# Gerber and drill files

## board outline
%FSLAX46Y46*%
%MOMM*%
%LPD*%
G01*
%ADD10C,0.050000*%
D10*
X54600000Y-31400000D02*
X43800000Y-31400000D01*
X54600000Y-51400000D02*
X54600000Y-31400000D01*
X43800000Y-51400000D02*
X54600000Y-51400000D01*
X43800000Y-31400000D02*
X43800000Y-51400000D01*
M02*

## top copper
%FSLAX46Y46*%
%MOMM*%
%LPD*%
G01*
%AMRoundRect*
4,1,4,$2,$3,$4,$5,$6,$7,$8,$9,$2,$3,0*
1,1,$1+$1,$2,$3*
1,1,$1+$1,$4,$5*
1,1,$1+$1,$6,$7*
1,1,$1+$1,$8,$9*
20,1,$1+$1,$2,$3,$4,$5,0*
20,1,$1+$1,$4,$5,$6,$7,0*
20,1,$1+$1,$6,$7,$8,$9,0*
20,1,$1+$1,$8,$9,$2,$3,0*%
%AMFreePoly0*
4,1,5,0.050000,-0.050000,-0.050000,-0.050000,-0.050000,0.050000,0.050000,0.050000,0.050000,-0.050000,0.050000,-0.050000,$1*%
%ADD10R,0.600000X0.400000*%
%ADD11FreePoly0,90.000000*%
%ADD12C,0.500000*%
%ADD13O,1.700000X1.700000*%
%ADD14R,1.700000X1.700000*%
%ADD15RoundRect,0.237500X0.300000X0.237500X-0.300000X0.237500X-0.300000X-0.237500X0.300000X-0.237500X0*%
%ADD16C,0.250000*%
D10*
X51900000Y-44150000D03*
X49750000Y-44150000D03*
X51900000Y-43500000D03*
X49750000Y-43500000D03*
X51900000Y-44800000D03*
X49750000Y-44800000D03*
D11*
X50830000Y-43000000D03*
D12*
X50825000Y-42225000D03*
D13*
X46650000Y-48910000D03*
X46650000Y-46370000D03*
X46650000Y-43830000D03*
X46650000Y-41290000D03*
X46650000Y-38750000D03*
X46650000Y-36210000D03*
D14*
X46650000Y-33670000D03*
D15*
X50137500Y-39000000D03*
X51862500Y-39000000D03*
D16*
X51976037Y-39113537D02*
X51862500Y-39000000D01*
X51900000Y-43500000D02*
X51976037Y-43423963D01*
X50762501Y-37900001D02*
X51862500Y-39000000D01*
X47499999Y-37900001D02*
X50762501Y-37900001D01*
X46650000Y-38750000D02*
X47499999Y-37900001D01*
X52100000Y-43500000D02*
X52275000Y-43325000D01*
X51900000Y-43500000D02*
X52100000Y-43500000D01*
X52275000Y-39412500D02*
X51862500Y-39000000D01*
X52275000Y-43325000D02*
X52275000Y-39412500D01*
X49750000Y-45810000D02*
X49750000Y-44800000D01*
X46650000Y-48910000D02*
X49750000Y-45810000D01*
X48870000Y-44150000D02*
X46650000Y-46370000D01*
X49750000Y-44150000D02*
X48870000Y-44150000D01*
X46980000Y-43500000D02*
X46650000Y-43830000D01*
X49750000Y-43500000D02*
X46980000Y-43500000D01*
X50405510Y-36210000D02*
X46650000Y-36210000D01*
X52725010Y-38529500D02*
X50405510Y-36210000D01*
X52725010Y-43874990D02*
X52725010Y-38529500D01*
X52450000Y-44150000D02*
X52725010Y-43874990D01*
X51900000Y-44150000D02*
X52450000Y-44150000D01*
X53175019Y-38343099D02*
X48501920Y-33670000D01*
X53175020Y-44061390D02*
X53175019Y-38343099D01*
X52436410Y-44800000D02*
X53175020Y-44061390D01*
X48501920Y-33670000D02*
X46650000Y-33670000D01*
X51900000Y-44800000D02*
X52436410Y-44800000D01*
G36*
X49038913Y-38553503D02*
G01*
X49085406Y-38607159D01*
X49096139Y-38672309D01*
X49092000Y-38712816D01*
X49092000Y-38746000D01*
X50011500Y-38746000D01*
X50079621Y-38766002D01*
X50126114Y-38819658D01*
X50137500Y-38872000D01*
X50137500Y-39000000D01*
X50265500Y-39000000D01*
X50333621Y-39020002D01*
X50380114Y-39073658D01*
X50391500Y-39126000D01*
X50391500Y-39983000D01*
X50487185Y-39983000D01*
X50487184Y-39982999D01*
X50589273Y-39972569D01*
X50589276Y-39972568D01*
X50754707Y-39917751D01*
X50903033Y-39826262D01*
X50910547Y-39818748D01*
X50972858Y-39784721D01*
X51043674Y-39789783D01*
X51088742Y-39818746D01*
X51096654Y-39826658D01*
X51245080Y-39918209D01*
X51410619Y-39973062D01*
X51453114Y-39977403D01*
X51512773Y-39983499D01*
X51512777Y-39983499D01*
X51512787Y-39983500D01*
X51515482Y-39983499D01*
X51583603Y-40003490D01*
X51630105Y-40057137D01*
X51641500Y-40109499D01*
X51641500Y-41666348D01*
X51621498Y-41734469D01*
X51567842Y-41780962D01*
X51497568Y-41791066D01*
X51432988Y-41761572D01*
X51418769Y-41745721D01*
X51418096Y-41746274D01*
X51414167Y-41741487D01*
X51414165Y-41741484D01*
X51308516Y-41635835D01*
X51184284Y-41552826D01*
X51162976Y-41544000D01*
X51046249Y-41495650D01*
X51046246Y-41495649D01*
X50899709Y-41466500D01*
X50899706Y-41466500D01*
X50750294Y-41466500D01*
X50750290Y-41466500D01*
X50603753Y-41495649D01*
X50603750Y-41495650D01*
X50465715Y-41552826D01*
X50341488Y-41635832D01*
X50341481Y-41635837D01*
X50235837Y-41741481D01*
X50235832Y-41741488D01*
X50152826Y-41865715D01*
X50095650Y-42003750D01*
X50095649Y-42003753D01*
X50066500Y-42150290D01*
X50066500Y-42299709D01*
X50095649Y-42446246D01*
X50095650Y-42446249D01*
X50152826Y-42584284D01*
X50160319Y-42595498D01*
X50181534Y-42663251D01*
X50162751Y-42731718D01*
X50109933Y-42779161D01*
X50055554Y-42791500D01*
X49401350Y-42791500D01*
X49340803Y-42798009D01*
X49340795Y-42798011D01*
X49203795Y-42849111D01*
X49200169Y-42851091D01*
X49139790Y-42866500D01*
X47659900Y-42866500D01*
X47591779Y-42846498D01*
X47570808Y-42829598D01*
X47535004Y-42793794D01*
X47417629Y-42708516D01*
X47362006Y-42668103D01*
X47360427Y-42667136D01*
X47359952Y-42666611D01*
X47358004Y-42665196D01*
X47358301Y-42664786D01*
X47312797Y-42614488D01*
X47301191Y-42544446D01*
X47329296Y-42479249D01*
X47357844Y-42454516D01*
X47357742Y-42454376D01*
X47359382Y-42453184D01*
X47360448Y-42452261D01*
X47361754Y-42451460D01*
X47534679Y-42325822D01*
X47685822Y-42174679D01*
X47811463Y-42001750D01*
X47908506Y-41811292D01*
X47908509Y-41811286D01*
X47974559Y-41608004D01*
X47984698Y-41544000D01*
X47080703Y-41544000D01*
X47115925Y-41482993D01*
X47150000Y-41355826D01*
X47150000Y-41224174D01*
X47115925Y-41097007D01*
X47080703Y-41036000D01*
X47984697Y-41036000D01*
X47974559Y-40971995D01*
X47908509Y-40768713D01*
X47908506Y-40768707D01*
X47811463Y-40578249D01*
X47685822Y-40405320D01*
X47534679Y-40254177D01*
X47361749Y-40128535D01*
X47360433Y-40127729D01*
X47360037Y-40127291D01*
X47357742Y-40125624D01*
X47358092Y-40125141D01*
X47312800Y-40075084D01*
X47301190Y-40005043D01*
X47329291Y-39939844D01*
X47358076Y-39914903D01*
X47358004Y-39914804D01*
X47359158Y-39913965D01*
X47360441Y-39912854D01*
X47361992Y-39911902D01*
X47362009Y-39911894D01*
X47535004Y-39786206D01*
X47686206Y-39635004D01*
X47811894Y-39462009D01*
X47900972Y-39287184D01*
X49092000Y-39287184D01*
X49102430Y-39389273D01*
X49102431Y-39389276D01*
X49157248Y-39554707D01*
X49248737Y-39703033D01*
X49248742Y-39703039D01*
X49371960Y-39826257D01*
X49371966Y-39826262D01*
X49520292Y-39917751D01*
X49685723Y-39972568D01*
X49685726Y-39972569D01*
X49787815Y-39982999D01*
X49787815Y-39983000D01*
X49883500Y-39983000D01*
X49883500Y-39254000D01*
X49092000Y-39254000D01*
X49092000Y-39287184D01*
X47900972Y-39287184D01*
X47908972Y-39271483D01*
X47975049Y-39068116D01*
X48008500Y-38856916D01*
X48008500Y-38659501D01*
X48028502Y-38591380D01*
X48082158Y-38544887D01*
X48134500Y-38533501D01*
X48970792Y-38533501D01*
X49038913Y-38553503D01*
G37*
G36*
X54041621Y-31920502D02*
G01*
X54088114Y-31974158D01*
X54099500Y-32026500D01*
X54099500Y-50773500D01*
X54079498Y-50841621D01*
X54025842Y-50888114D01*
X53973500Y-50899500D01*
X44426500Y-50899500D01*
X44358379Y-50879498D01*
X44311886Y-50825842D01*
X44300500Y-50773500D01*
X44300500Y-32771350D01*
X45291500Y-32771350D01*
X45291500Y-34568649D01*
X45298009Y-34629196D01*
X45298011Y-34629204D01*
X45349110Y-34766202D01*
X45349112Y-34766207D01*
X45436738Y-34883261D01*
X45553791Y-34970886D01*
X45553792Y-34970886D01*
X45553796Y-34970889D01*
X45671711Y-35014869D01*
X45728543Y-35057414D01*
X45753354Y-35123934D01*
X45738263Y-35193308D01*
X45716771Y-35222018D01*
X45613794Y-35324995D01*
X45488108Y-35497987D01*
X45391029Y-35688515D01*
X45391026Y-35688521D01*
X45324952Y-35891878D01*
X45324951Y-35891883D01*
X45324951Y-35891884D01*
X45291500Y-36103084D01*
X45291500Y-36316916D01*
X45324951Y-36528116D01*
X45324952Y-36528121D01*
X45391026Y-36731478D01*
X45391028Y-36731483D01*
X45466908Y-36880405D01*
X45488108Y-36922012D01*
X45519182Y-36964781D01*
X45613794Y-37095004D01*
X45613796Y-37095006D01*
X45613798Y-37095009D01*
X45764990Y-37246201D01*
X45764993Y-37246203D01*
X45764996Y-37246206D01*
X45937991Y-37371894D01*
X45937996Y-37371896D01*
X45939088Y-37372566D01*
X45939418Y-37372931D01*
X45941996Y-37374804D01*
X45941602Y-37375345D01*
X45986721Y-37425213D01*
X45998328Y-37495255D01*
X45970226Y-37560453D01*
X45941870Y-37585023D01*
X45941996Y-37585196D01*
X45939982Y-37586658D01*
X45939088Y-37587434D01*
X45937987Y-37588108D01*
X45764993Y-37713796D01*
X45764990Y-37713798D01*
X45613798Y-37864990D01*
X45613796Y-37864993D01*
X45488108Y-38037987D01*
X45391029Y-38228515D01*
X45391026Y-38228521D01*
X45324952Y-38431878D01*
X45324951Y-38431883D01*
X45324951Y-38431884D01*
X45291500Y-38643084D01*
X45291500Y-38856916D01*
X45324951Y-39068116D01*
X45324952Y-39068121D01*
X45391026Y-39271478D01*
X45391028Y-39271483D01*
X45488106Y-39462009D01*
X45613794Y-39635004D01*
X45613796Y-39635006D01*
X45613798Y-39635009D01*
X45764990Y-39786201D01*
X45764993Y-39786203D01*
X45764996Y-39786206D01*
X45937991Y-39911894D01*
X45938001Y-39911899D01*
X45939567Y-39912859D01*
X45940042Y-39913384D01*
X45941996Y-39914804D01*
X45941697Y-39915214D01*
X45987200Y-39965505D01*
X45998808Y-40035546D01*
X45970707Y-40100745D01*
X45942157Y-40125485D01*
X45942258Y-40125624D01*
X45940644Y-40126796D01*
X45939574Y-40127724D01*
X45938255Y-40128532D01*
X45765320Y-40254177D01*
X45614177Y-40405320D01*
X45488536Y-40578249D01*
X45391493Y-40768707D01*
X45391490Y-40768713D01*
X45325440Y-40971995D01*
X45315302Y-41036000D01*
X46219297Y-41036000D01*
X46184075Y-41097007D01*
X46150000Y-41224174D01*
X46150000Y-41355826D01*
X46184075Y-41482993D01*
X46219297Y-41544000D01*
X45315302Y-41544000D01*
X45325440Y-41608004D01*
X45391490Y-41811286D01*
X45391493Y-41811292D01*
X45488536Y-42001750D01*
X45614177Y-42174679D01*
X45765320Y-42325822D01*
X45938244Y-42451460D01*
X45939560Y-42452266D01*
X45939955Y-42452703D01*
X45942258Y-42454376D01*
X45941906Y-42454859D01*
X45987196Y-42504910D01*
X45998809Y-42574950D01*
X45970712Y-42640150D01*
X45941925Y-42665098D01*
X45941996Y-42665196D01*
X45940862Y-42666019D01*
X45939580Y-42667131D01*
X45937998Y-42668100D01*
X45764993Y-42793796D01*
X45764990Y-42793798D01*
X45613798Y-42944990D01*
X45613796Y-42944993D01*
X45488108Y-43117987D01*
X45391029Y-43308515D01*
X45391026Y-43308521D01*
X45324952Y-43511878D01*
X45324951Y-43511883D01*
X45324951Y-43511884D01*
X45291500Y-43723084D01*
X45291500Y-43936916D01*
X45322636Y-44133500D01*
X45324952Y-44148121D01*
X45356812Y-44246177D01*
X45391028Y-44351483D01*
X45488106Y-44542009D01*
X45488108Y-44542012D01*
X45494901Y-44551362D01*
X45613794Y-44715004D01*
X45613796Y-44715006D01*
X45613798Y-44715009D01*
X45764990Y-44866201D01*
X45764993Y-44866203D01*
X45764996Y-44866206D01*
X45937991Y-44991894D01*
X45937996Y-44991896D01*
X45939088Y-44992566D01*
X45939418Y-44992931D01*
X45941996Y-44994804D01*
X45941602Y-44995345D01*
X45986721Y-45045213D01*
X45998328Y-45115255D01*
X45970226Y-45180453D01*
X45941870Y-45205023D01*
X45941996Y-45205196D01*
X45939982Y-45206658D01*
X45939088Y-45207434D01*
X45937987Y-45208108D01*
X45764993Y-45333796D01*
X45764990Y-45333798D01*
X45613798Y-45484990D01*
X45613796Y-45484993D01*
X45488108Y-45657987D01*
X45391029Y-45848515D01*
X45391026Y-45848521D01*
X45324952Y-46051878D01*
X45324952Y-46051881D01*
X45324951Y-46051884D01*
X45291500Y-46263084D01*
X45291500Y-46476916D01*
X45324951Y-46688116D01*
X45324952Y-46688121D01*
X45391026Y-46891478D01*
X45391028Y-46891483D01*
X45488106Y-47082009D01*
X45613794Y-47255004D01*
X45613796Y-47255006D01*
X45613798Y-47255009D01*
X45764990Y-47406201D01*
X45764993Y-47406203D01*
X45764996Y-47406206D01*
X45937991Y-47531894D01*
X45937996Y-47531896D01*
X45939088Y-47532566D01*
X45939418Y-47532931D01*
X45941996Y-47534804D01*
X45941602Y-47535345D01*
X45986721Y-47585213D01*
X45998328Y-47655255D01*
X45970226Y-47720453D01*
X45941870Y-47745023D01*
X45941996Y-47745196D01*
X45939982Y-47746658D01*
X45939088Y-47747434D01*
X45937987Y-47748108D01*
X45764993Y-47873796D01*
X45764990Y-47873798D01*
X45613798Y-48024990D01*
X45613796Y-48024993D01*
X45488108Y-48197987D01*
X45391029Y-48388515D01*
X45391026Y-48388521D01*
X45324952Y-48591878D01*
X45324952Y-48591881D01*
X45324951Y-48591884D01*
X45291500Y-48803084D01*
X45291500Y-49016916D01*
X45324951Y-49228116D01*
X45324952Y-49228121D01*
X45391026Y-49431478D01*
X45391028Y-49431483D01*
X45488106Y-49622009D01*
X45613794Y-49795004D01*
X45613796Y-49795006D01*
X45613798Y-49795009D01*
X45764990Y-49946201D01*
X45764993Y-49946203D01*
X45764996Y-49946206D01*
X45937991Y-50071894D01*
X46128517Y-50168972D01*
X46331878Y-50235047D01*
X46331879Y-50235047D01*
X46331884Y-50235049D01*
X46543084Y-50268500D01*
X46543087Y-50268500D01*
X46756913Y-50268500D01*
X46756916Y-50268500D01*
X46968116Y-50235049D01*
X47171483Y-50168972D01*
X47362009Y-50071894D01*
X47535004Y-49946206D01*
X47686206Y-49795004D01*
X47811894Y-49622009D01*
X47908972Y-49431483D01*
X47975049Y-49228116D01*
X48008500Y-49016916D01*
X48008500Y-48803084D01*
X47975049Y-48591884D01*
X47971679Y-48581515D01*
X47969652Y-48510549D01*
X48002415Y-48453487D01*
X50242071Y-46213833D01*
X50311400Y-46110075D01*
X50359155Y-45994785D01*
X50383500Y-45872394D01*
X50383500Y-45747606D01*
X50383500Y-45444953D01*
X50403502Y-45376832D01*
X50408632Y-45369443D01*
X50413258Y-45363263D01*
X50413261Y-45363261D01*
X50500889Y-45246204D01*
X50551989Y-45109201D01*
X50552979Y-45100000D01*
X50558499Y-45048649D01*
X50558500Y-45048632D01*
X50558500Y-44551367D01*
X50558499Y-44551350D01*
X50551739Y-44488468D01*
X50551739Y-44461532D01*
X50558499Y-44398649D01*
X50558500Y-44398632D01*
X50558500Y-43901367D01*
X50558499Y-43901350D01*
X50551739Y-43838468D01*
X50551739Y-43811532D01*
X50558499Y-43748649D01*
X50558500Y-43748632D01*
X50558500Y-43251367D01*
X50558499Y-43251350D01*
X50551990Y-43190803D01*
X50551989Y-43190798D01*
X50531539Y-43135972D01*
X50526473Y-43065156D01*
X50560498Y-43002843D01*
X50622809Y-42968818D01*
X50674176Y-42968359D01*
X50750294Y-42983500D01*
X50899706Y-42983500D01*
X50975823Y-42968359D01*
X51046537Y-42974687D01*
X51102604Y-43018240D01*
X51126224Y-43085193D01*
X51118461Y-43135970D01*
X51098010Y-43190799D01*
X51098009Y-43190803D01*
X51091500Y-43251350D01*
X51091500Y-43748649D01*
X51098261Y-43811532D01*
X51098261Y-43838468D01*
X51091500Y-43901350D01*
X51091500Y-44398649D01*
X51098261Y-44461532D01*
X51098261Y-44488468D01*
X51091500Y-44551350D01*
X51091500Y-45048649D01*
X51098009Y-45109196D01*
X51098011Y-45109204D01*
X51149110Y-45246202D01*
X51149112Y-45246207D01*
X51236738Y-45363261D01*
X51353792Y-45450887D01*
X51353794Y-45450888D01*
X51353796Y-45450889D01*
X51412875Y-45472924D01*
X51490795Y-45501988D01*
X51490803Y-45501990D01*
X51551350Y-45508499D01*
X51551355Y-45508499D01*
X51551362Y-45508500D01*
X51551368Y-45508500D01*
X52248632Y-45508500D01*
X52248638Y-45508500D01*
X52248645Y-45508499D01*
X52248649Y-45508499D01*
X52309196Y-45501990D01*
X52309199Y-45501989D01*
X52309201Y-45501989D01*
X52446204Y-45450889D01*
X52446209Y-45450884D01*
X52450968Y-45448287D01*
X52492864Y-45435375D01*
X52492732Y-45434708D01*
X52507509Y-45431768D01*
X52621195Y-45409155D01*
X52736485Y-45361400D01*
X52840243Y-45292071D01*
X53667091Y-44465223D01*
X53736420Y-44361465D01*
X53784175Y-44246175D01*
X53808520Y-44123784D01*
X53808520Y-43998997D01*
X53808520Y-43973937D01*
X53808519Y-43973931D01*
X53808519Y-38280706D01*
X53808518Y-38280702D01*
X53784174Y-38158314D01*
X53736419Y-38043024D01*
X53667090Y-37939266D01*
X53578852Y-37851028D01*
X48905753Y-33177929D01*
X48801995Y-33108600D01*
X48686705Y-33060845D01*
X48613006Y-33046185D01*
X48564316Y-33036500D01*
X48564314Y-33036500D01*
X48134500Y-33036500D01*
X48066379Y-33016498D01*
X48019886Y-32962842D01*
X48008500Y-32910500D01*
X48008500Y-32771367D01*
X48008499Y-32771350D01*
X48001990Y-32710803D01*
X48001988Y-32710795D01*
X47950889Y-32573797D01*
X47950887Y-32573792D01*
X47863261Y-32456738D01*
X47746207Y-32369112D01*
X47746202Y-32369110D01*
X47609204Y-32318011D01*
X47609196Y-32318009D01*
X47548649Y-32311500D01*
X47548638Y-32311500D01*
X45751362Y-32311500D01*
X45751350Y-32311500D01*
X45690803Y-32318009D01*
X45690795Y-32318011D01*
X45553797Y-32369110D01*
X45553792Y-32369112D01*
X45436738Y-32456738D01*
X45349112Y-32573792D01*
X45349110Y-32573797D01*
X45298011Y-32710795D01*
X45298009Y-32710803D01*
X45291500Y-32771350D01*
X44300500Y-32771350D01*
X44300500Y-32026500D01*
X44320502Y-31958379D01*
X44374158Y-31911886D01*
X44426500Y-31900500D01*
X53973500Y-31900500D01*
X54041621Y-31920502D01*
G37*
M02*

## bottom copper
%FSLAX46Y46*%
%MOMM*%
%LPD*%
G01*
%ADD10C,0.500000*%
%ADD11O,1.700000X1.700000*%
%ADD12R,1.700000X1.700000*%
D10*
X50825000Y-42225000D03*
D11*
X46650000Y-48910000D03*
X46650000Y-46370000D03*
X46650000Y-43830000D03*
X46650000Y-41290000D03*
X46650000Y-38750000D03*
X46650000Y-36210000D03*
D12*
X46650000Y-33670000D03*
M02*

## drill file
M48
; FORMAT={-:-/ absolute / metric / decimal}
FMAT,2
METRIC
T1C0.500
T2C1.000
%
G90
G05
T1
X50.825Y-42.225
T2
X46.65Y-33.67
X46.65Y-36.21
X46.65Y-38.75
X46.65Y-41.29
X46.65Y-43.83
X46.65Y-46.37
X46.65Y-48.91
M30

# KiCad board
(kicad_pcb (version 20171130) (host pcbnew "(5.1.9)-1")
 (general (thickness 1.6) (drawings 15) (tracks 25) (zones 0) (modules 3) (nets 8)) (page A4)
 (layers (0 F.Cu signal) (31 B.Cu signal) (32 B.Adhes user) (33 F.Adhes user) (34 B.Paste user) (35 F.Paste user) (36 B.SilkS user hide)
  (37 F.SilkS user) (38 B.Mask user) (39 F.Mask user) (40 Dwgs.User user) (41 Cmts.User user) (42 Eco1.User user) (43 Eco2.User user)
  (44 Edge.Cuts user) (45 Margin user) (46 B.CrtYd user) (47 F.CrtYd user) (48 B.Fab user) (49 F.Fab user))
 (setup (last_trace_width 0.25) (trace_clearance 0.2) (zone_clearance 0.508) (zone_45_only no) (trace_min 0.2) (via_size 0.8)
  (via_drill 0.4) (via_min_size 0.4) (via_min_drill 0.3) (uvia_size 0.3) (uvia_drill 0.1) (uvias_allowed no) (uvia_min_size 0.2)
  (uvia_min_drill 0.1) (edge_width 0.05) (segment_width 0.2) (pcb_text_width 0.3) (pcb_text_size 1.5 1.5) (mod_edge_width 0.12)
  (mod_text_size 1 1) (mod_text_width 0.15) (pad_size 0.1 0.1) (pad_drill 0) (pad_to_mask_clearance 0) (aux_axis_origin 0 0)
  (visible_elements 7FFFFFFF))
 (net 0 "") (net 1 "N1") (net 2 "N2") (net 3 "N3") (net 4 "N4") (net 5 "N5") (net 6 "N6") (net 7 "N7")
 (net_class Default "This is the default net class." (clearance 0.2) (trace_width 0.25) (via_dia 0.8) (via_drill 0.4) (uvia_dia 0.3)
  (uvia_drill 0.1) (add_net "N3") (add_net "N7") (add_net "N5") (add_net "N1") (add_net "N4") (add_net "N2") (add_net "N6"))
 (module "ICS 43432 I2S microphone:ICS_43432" (layer F.Cu) (at 50.8 43.2 90)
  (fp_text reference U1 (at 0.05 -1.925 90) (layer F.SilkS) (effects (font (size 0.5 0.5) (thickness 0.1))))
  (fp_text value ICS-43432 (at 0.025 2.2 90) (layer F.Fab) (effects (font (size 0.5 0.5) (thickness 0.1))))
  (pad 2 smd rect (at -0.95 1.1 90) (size 0.4 0.6) (layers F.Cu F.Paste F.Mask) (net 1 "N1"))
  (pad 6 smd rect (at -0.95 -1.05 90) (size 0.4 0.6) (layers F.Cu F.Paste F.Mask) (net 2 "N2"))
  (pad 3 smd rect (at -0.3 1.1 90) (size 0.4 0.6) (layers F.Cu F.Paste F.Mask) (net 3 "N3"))
  (pad 5 smd rect (at -0.3 -1.05 90) (size 0.4 0.6) (layers F.Cu F.Paste F.Mask) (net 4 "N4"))
  (pad 1 smd rect (at -1.6 1.1 90) (size 0.4 0.6) (layers F.Cu F.Paste F.Mask) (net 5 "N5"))
  (pad 7 smd rect (at -1.6 -1.05 90) (size 0.4 0.6) (layers F.Cu F.Paste F.Mask) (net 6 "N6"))
  (pad 4 smd custom (at 0.2 0.03 90) (size 0.1 0.1) (layers F.Cu F.Paste F.Mask) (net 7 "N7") (zone_connect 2)
   (options (clearance outline) (anchor rect)) (primitives))
  (pad 12 thru_hole circle (at 0.975 0.025 90) (size 0.5 0.5) (drill 0.5) (layers *.Cu *.Mask) (zone_connect 0)))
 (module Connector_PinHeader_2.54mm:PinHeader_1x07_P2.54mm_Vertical (layer B.Cu) (at 46.65 33.67 180)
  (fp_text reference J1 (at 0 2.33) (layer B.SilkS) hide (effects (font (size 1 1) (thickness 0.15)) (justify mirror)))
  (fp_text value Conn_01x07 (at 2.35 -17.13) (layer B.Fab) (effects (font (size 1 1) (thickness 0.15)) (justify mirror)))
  (pad 7 thru_hole oval (at 0 -15.24 180) (size 1.7 1.7) (drill 1) (layers *.Cu *.Mask) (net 6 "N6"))
  (pad 6 thru_hole oval (at 0 -12.7 180) (size 1.7 1.7) (drill 1) (layers *.Cu *.Mask) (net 2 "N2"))
  (pad 5 thru_hole oval (at 0 -10.16 180) (size 1.7 1.7) (drill 1) (layers *.Cu *.Mask) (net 4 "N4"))
  (pad 4 thru_hole oval (at 0 -7.62 180) (size 1.7 1.7) (drill 1) (layers *.Cu *.Mask) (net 7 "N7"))
  (pad 3 thru_hole oval (at 0 -5.08 180) (size 1.7 1.7) (drill 1) (layers *.Cu *.Mask) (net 3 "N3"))
  (pad 2 thru_hole oval (at 0 -2.54 180) (size 1.7 1.7) (drill 1) (layers *.Cu *.Mask) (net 1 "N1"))
  (pad 1 thru_hole rect (at 0 0 180) (size 1.7 1.7) (drill 1) (layers *.Cu *.Mask) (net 5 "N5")))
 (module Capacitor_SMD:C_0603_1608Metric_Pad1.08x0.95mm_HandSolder (layer F.Cu) (at 51 39 180)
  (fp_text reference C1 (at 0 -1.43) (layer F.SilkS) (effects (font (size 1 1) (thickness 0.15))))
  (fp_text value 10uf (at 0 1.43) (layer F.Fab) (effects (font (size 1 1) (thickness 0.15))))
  (pad 2 smd roundrect (at 0.8625 0 180) (size 1.075 0.95) (layers F.Cu F.Paste F.Mask) (roundrect_rratio 0.25) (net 7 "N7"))
  (pad 1 smd roundrect (at -0.8625 0 180) (size 1.075 0.95) (layers F.Cu F.Paste F.Mask) (roundrect_rratio 0.25) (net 3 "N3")))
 (gr_line (start 54.6 31.4) (end 43.8 31.4) (layer Edge.Cuts) (width 0.05))
 (gr_line (start 54.6 51.4) (end 54.6 31.4) (layer Edge.Cuts) (width 0.05))
 (gr_line (start 43.8 51.4) (end 54.6 51.4) (layer Edge.Cuts) (width 0.05))
 (gr_line (start 43.8 31.4) (end 43.8 51.4) (layer Edge.Cuts) (width 0.05))
 (segment (start 51.976037 39.113537) (end 51.8625 39) (width 0.25) (layer F.Cu) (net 3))
 (segment (start 51.9 43.5) (end 51.976037 43.423963) (width 0.25) (layer F.Cu) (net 3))
 (segment (start 50.762501 37.900001) (end 51.8625 39) (width 0.25) (layer F.Cu) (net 3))
 (segment (start 47.499999 37.900001) (end 50.762501 37.900001) (width 0.25) (layer F.Cu) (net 3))
 (segment (start 46.65 38.75) (end 47.499999 37.900001) (width 0.25) (layer F.Cu) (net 3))
 (segment (start 52.1 43.5) (end 52.275 43.325) (width 0.25) (layer F.Cu) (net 3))
 (segment (start 51.9 43.5) (end 52.1 43.5) (width 0.25) (layer F.Cu) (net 3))
 (segment (start 52.275 39.4125) (end 51.8625 39) (width 0.25) (layer F.Cu) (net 3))
 (segment (start 52.275 43.325) (end 52.275 39.4125) (width 0.25) (layer F.Cu) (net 3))
 (segment (start 49.75 45.81) (end 49.75 44.8) (width 0.25) (layer F.Cu) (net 6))
 (segment (start 46.65 48.91) (end 49.75 45.81) (width 0.25) (layer F.Cu) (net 6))
 (segment (start 48.87 44.15) (end 46.65 46.37) (width 0.25) (layer F.Cu) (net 2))
 (segment (start 49.75 44.15) (end 48.87 44.15) (width 0.25) (layer F.Cu) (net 2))
 (segment (start 46.98 43.5) (end 46.65 43.83) (width 0.25) (layer F.Cu) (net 4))
 (segment (start 49.75 43.5) (end 46.98 43.5) (width 0.25) (layer F.Cu) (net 4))
 (segment (start 50.40551 36.21) (end 46.65 36.21) (width 0.25) (layer F.Cu) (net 1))
 (segment (start 52.72501 38.5295) (end 50.40551 36.21) (width 0.25) (layer F.Cu) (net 1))
 (segment (start 52.72501 43.87499) (end 52.72501 38.5295) (width 0.25) (layer F.Cu) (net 1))
 (segment (start 52.45 44.15) (end 52.72501 43.87499) (width 0.25) (layer F.Cu) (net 1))
 (segment (start 51.9 44.15) (end 52.45 44.15) (width 0.25) (layer F.Cu) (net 1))
 (segment (start 53.175019 38.343099) (end 48.50192 33.67) (width 0.25) (layer F.Cu) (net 5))
 (segment (start 53.17502 44.06139) (end 53.175019 38.343099) (width 0.25) (layer F.Cu) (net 5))
 (segment (start 52.43641 44.8) (end 53.17502 44.06139) (width 0.25) (layer F.Cu) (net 5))
 (segment (start 48.50192 33.67) (end 46.65 33.67) (width 0.25) (layer F.Cu) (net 5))
 (segment (start 51.9 44.8) (end 52.43641 44.8) (width 0.25) (layer F.Cu) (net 5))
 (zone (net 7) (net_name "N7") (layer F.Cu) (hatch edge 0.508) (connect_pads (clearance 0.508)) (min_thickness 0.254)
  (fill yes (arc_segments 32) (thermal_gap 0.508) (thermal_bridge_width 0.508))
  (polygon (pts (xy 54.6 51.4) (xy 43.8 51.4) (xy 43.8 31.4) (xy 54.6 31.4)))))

